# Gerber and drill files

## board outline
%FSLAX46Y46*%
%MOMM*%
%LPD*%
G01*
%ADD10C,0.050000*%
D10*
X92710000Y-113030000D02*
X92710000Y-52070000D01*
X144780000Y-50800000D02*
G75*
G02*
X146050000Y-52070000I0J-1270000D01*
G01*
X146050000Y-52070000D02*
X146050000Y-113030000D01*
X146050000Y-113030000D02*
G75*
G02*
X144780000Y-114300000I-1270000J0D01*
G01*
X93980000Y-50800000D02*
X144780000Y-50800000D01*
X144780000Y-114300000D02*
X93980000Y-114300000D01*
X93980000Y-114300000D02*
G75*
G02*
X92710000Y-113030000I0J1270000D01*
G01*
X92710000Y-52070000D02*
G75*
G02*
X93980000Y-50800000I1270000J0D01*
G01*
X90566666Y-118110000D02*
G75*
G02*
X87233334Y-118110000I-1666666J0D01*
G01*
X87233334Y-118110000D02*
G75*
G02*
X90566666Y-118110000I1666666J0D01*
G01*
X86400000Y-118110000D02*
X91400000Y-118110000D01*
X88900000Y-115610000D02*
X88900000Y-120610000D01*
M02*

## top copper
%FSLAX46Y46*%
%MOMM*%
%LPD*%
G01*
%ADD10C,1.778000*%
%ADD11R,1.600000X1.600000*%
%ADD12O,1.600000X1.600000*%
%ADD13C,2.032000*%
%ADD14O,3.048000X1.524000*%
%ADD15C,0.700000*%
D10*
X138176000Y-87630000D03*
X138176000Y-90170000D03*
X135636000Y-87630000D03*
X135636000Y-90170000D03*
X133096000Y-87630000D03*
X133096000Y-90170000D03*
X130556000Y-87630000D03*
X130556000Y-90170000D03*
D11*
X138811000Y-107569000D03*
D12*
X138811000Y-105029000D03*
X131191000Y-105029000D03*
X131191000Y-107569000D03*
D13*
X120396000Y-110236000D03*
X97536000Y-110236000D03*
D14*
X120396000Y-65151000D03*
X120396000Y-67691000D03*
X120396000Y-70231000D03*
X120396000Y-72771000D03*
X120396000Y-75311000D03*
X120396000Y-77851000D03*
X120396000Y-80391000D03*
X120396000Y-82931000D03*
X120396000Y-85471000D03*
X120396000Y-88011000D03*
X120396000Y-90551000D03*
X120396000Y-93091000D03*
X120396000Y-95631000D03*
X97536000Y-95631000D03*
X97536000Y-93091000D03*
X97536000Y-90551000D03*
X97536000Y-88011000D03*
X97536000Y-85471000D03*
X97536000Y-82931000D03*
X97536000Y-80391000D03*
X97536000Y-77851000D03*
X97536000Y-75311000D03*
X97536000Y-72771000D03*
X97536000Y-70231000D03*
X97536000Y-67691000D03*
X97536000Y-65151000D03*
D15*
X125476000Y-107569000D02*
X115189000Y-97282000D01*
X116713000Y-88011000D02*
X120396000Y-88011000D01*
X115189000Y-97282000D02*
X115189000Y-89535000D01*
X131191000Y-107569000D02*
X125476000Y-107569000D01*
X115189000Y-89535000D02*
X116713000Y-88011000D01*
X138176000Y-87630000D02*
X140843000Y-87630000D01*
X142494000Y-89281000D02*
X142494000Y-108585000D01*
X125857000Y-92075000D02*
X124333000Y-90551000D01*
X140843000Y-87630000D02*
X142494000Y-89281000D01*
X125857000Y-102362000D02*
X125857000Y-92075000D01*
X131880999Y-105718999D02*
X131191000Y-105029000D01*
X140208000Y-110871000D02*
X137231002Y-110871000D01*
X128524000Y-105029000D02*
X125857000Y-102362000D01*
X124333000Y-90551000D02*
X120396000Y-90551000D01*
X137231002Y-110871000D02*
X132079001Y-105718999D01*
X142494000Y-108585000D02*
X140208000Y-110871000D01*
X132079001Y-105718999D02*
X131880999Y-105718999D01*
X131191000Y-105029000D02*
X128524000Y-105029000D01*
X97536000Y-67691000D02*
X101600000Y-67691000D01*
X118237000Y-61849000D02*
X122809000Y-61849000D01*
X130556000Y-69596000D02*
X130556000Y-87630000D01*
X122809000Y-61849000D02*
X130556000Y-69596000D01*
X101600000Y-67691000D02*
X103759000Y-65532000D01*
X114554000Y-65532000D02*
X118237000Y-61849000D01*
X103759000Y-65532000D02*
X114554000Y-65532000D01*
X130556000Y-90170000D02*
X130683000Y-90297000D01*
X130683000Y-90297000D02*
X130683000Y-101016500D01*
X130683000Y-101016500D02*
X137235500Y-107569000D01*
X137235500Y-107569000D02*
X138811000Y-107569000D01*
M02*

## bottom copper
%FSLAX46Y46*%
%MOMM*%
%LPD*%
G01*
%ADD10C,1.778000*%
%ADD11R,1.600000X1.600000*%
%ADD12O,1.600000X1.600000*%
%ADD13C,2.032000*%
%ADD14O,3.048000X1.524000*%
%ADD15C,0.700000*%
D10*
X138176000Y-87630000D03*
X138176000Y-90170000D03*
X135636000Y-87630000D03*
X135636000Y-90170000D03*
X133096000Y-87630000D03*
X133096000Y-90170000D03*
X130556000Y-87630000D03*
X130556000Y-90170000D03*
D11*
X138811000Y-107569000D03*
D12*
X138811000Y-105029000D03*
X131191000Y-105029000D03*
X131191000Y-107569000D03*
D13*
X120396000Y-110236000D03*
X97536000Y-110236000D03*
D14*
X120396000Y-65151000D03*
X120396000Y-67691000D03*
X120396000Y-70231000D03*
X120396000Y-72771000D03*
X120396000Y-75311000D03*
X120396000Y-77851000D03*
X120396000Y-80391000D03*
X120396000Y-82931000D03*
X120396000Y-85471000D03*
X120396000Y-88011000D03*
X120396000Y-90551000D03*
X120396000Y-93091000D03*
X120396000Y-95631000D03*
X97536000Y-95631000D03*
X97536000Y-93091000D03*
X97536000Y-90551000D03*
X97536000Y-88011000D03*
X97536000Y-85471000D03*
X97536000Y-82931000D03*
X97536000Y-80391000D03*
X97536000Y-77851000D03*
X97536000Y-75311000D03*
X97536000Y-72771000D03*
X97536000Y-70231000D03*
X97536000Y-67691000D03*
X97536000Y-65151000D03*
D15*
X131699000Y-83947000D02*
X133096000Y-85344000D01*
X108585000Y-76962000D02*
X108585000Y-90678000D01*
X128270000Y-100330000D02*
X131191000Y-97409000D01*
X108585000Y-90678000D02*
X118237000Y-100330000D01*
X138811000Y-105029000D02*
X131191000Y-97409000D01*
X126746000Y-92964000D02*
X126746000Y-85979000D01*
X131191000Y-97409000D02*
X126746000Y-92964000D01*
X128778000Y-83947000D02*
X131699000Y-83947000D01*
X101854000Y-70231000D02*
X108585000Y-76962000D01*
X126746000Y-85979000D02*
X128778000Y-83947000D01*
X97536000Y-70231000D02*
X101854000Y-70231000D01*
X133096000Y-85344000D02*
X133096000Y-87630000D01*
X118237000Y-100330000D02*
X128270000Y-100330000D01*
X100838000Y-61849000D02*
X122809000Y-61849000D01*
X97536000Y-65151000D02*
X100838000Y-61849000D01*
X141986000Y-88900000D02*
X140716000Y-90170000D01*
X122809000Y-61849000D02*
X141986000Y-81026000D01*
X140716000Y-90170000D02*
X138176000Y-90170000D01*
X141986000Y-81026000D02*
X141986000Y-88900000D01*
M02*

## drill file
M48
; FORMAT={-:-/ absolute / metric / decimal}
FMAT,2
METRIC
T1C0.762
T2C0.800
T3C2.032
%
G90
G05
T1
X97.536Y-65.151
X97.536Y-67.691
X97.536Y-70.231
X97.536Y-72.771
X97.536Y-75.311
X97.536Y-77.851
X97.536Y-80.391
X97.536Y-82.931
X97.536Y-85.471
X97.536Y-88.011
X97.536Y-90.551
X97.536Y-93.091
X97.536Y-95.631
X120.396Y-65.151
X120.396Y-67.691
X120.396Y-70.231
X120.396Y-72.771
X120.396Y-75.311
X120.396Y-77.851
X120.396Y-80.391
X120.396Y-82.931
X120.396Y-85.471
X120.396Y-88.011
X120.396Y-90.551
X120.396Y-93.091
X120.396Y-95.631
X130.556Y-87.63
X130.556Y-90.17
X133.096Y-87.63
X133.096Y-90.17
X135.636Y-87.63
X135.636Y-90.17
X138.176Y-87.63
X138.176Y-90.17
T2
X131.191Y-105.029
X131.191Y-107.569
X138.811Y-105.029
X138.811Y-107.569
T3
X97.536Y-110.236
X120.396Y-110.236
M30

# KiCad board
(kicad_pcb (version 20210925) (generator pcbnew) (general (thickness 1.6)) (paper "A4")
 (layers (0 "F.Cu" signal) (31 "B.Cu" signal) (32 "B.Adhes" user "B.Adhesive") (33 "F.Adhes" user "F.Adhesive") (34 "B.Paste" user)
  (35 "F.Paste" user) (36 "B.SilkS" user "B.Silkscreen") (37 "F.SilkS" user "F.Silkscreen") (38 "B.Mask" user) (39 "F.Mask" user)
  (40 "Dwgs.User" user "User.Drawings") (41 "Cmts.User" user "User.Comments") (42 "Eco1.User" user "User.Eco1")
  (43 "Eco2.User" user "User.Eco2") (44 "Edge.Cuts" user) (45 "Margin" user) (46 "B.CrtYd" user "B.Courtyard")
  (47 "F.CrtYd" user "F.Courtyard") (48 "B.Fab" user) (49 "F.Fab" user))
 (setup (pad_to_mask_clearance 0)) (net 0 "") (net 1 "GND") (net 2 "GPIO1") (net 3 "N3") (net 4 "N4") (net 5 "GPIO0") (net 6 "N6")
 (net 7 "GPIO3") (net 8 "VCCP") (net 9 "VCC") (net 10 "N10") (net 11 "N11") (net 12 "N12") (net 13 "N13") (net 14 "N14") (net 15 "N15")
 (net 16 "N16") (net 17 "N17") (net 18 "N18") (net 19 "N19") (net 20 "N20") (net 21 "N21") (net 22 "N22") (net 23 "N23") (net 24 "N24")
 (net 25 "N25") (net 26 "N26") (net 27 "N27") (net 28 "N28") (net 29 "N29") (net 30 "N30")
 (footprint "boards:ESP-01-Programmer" (layer "F.Cu") (at 134.366 74.295)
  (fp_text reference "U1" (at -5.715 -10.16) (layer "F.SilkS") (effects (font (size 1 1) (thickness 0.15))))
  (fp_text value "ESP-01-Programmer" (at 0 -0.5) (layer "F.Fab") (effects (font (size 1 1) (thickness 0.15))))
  (pad "1" thru_hole circle locked (at 3.81 13.335) (size 1.778 1.778) (drill 0.762) (layers *.Cu *.Mask) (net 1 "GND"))
  (pad "2" thru_hole circle locked (at 3.81 15.875) (size 1.778 1.778) (drill 0.762) (layers *.Cu *.Mask) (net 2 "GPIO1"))
  (pad "3" thru_hole circle locked (at 1.27 13.335) (size 1.778 1.778) (drill 0.762) (layers *.Cu *.Mask) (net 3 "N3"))
  (pad "4" thru_hole circle locked (at 1.27 15.875) (size 1.778 1.778) (drill 0.762) (layers *.Cu *.Mask) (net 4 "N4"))
  (pad "5" thru_hole circle locked (at -1.27 13.335) (size 1.778 1.778) (drill 0.762) (layers *.Cu *.Mask) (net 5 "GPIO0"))
  (pad "6" thru_hole circle locked (at -1.27 15.875) (size 1.778 1.778) (drill 0.762) (layers *.Cu *.Mask) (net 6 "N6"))
  (pad "7" thru_hole circle locked (at -3.81 13.335) (size 1.778 1.778) (drill 0.762) (layers *.Cu *.Mask) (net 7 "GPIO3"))
  (pad "8" thru_hole circle locked (at -3.81 15.875) (size 1.778 1.778) (drill 0.762) (layers *.Cu *.Mask) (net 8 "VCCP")))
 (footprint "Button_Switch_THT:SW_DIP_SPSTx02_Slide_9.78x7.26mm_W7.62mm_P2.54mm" (layer "F.Cu") (at 138.811 107.569 180)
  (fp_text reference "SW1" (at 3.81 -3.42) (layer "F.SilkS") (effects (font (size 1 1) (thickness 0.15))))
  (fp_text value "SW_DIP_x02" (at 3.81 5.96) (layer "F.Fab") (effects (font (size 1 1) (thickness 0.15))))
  (pad "1" thru_hole rect locked (at 0 0 180) (size 1.6 1.6) (drill 0.8) (layers *.Cu *.Mask) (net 8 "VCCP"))
  (pad "2" thru_hole oval locked (at 0 2.54 180) (size 1.6 1.6) (drill 0.8) (layers *.Cu *.Mask) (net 5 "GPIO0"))
  (pad "3" thru_hole oval locked (at 7.62 2.54 180) (size 1.6 1.6) (drill 0.8) (layers *.Cu *.Mask) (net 1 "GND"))
  (pad "4" thru_hole oval locked (at 7.62 0 180) (size 1.6 1.6) (drill 0.8) (layers *.Cu *.Mask) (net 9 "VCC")))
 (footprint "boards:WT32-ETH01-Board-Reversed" (layer "F.Cu") (at 108.966 84.201)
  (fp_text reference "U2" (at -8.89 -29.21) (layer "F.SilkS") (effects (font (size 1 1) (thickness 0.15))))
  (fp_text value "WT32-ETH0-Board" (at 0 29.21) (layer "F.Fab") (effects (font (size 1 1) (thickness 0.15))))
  (pad "" thru_hole circle locked (at 11.43 26.035) (size 2.032 2.032) (drill 2.032) (layers *.Mask "F.Cu"))
  (pad "" thru_hole circle locked (at -11.43 26.035) (size 2.032 2.032) (drill 2.032) (layers *.Mask "F.Cu"))
  (pad "1" thru_hole oval locked (at 11.43 -19.05) (size 3.048 1.524) (drill 0.762) (layers *.Cu *.Mask) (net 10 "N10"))
  (pad "2" thru_hole oval locked (at 11.43 -16.51) (size 3.048 1.524) (drill 0.762) (layers *.Cu *.Mask) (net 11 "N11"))
  (pad "3" thru_hole oval locked (at 11.43 -13.97) (size 3.048 1.524) (drill 0.762) (layers *.Cu *.Mask) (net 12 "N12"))
  (pad "4" thru_hole oval locked (at 11.43 -11.43) (size 3.048 1.524) (drill 0.762) (layers *.Cu *.Mask) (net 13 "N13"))
  (pad "5" thru_hole oval locked (at 11.43 -8.89) (size 3.048 1.524) (drill 0.762) (layers *.Cu *.Mask) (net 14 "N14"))
  (pad "6" thru_hole oval locked (at 11.43 -6.35) (size 3.048 1.524) (drill 0.762) (layers *.Cu *.Mask) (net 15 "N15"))
  (pad "7" thru_hole oval locked (at 11.43 -3.81) (size 3.048 1.524) (drill 0.762) (layers *.Cu *.Mask) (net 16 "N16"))
  (pad "8" thru_hole oval locked (at 11.43 -1.27) (size 3.048 1.524) (drill 0.762) (layers *.Cu *.Mask) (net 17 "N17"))
  (pad "9" thru_hole oval locked (at 11.43 1.27) (size 3.048 1.524) (drill 0.762) (layers *.Cu *.Mask) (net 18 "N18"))
  (pad "10" thru_hole oval locked (at 11.43 3.81) (size 3.048 1.524) (drill 0.762) (layers *.Cu *.Mask) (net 9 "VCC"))
  (pad "11" thru_hole oval locked (at 11.43 6.35) (size 3.048 1.524) (drill 0.762) (layers *.Cu *.Mask) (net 1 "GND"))
  (pad "12" thru_hole oval locked (at 11.43 8.89) (size 3.048 1.524) (drill 0.762) (layers *.Cu *.Mask) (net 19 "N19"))
  (pad "13" thru_hole oval locked (at 11.43 11.43) (size 3.048 1.524) (drill 0.762) (layers *.Cu *.Mask) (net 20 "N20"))
  (pad "14" thru_hole oval locked (at -11.43 11.43) (size 3.048 1.524) (drill 0.762) (layers *.Cu *.Mask) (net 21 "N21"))
  (pad "15" thru_hole oval locked (at -11.43 8.89) (size 3.048 1.524) (drill 0.762) (layers *.Cu *.Mask) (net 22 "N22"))
  (pad "16" thru_hole oval locked (at -11.43 6.35) (size 3.048 1.524) (drill 0.762) (layers *.Cu *.Mask) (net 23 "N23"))
  (pad "17" thru_hole oval locked (at -11.43 3.81) (size 3.048 1.524) (drill 0.762) (layers *.Cu *.Mask) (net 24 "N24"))
  (pad "18" thru_hole oval locked (at -11.43 1.27) (size 3.048 1.524) (drill 0.762) (layers *.Cu *.Mask) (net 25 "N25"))
  (pad "19" thru_hole oval locked (at -11.43 -1.27) (size 3.048 1.524) (drill 0.762) (layers *.Cu *.Mask) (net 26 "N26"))
  (pad "20" thru_hole oval locked (at -11.43 -3.81) (size 3.048 1.524) (drill 0.762) (layers *.Cu *.Mask) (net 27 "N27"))
  (pad "21" thru_hole oval locked (at -11.43 -6.35) (size 3.048 1.524) (drill 0.762) (layers *.Cu *.Mask) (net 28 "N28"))
  (pad "22" thru_hole oval locked (at -11.43 -8.89) (size 3.048 1.524) (drill 0.762) (layers *.Cu *.Mask) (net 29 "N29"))
  (pad "23" thru_hole oval locked (at -11.43 -11.43) (size 3.048 1.524) (drill 0.762) (layers *.Cu *.Mask) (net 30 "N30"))
  (pad "24" thru_hole oval locked (at -11.43 -13.97) (size 3.048 1.524) (drill 0.762) (layers *.Cu *.Mask) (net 5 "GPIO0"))
  (pad "25" thru_hole oval locked (at -11.43 -16.51) (size 3.048 1.524) (drill 0.762) (layers *.Cu *.Mask) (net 7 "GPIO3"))
  (pad "26" thru_hole oval locked (at -11.43 -19.05) (size 3.048 1.524) (drill 0.762) (layers *.Cu *.Mask) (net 2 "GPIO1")))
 (gr_line (start 92.71 113.03) (end 92.71 52.07) (layer "Edge.Cuts") (width 0.05))
 (gr_arc (start 144.78 52.07) (end 146.05 52.07) (angle -90) (layer "Edge.Cuts") (width 0.05))
 (gr_line (start 146.05 52.07) (end 146.05 113.03) (layer "Edge.Cuts") (width 0.05))
 (gr_arc (start 144.78 113.03) (end 144.78 114.3) (angle -90) (layer "Edge.Cuts") (width 0.05))
 (gr_line (start 93.98 50.8) (end 144.78 50.8) (layer "Edge.Cuts") (width 0.05))
 (gr_line (start 144.78 114.3) (end 93.98 114.3) (layer "Edge.Cuts") (width 0.05))
 (gr_arc (start 93.98 113.03) (end 92.71 113.03) (angle -90) (layer "Edge.Cuts") (width 0.05))
 (gr_arc (start 93.98 52.07) (end 93.98 50.8) (angle -90) (layer "Edge.Cuts") (width 0.05))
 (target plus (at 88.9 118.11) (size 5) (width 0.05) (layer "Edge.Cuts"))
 (segment (start 125.476 107.569) (end 115.189 97.282) (width 0.7) (layer "F.Cu") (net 9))
 (segment (start 116.713 88.011) (end 120.396 88.011) (width 0.7) (layer "F.Cu") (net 9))
 (segment (start 115.189 97.282) (end 115.189 89.535) (width 0.7) (layer "F.Cu") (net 9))
 (segment (start 131.191 107.569) (end 125.476 107.569) (width 0.7) (layer "F.Cu") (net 9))
 (segment (start 115.189 89.535) (end 116.713 88.011) (width 0.7) (layer "F.Cu") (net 9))
 (segment (start 131.699 83.947) (end 133.096 85.344) (width 0.7) (layer "B.Cu") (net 5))
 (segment (start 108.585 76.962) (end 108.585 90.678) (width 0.7) (layer "B.Cu") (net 5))
 (segment (start 128.27 100.33) (end 131.191 97.409) (width 0.7) (layer "B.Cu") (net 5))
 (segment (start 108.585 90.678) (end 118.237 100.33) (width 0.7) (layer "B.Cu") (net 5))
 (segment (start 138.811 105.029) (end 131.191 97.409) (width 0.7) (layer "B.Cu") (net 5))
 (segment (start 126.746 92.964) (end 126.746 85.979) (width 0.7) (layer "B.Cu") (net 5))
 (segment (start 131.191 97.409) (end 126.746 92.964) (width 0.7) (layer "B.Cu") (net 5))
 (segment (start 128.778 83.947) (end 131.699 83.947) (width 0.7) (layer "B.Cu") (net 5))
 (segment (start 101.854 70.231) (end 108.585 76.962) (width 0.7) (layer "B.Cu") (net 5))
 (segment (start 126.746 85.979) (end 128.778 83.947) (width 0.7) (layer "B.Cu") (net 5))
 (segment (start 97.536 70.231) (end 101.854 70.231) (width 0.7) (layer "B.Cu") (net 5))
 (segment (start 133.096 85.344) (end 133.096 87.63) (width 0.7) (layer "B.Cu") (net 5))
 (segment (start 118.237 100.33) (end 128.27 100.33) (width 0.7) (layer "B.Cu") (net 5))
 (segment (start 138.176 87.63) (end 140.843 87.63) (width 0.7) (layer "F.Cu") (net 1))
 (segment (start 142.494 89.281) (end 142.494 108.585) (width 0.7) (layer "F.Cu") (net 1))
 (segment (start 125.857 92.075) (end 124.333 90.551) (width 0.7) (layer "F.Cu") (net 1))
 (segment (start 140.843 87.63) (end 142.494 89.281) (width 0.7) (layer "F.Cu") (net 1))
 (segment (start 125.857 102.362) (end 125.857 92.075) (width 0.7) (layer "F.Cu") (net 1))
 (segment (start 131.880999 105.718999) (end 131.191 105.029) (width 0.7) (layer "F.Cu") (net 1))
 (segment (start 140.208 110.871) (end 137.231002 110.871) (width 0.7) (layer "F.Cu") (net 1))
 (segment (start 128.524 105.029) (end 125.857 102.362) (width 0.7) (layer "F.Cu") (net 1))
 (segment (start 124.333 90.551) (end 120.396 90.551) (width 0.7) (layer "F.Cu") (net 1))
 (segment (start 137.231002 110.871) (end 132.079001 105.718999) (width 0.7) (layer "F.Cu") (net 1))
 (segment (start 142.494 108.585) (end 140.208 110.871) (width 0.7) (layer "F.Cu") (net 1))
 (segment (start 132.079001 105.718999) (end 131.880999 105.718999) (width 0.7) (layer "F.Cu") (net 1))
 (segment (start 131.191 105.029) (end 128.524 105.029) (width 0.7) (layer "F.Cu") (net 1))
 (segment (start 97.536 67.691) (end 101.6 67.691) (width 0.7) (layer "F.Cu") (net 7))
 (segment (start 118.237 61.849) (end 122.809 61.849) (width 0.7) (layer "F.Cu") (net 7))
 (segment (start 130.556 69.596) (end 130.556 87.63) (width 0.7) (layer "F.Cu") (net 7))
 (segment (start 122.809 61.849) (end 130.556 69.596) (width 0.7) (layer "F.Cu") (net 7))
 (segment (start 101.6 67.691) (end 103.759 65.532) (width 0.7) (layer "F.Cu") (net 7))
 (segment (start 114.554 65.532) (end 118.237 61.849) (width 0.7) (layer "F.Cu") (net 7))
 (segment (start 103.759 65.532) (end 114.554 65.532) (width 0.7) (layer "F.Cu") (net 7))
 (segment (start 100.838 61.849) (end 122.809 61.849) (width 0.7) (layer "B.Cu") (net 2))
 (segment (start 97.536 65.151) (end 100.838 61.849) (width 0.7) (layer "B.Cu") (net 2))
 (segment (start 141.986 88.9) (end 140.716 90.17) (width 0.7) (layer "B.Cu") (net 2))
 (segment (start 122.809 61.849) (end 141.986 81.026) (width 0.7) (layer "B.Cu") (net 2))
 (segment (start 140.716 90.17) (end 138.176 90.17) (width 0.7) (layer "B.Cu") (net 2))
 (segment (start 141.986 81.026) (end 141.986 88.9) (width 0.7) (layer "B.Cu") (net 2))
 (segment (start 130.556 90.17) (end 130.683 90.297) (width 0.7) (layer "F.Cu") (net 8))
 (segment (start 130.683 90.297) (end 130.683 101.0165) (width 0.7) (layer "F.Cu") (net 8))
 (segment (start 130.683 101.0165) (end 137.2355 107.569) (width 0.7) (layer "F.Cu") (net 8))
 (segment (start 137.2355 107.569) (end 138.811 107.569) (width 0.7) (layer "F.Cu") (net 8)))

